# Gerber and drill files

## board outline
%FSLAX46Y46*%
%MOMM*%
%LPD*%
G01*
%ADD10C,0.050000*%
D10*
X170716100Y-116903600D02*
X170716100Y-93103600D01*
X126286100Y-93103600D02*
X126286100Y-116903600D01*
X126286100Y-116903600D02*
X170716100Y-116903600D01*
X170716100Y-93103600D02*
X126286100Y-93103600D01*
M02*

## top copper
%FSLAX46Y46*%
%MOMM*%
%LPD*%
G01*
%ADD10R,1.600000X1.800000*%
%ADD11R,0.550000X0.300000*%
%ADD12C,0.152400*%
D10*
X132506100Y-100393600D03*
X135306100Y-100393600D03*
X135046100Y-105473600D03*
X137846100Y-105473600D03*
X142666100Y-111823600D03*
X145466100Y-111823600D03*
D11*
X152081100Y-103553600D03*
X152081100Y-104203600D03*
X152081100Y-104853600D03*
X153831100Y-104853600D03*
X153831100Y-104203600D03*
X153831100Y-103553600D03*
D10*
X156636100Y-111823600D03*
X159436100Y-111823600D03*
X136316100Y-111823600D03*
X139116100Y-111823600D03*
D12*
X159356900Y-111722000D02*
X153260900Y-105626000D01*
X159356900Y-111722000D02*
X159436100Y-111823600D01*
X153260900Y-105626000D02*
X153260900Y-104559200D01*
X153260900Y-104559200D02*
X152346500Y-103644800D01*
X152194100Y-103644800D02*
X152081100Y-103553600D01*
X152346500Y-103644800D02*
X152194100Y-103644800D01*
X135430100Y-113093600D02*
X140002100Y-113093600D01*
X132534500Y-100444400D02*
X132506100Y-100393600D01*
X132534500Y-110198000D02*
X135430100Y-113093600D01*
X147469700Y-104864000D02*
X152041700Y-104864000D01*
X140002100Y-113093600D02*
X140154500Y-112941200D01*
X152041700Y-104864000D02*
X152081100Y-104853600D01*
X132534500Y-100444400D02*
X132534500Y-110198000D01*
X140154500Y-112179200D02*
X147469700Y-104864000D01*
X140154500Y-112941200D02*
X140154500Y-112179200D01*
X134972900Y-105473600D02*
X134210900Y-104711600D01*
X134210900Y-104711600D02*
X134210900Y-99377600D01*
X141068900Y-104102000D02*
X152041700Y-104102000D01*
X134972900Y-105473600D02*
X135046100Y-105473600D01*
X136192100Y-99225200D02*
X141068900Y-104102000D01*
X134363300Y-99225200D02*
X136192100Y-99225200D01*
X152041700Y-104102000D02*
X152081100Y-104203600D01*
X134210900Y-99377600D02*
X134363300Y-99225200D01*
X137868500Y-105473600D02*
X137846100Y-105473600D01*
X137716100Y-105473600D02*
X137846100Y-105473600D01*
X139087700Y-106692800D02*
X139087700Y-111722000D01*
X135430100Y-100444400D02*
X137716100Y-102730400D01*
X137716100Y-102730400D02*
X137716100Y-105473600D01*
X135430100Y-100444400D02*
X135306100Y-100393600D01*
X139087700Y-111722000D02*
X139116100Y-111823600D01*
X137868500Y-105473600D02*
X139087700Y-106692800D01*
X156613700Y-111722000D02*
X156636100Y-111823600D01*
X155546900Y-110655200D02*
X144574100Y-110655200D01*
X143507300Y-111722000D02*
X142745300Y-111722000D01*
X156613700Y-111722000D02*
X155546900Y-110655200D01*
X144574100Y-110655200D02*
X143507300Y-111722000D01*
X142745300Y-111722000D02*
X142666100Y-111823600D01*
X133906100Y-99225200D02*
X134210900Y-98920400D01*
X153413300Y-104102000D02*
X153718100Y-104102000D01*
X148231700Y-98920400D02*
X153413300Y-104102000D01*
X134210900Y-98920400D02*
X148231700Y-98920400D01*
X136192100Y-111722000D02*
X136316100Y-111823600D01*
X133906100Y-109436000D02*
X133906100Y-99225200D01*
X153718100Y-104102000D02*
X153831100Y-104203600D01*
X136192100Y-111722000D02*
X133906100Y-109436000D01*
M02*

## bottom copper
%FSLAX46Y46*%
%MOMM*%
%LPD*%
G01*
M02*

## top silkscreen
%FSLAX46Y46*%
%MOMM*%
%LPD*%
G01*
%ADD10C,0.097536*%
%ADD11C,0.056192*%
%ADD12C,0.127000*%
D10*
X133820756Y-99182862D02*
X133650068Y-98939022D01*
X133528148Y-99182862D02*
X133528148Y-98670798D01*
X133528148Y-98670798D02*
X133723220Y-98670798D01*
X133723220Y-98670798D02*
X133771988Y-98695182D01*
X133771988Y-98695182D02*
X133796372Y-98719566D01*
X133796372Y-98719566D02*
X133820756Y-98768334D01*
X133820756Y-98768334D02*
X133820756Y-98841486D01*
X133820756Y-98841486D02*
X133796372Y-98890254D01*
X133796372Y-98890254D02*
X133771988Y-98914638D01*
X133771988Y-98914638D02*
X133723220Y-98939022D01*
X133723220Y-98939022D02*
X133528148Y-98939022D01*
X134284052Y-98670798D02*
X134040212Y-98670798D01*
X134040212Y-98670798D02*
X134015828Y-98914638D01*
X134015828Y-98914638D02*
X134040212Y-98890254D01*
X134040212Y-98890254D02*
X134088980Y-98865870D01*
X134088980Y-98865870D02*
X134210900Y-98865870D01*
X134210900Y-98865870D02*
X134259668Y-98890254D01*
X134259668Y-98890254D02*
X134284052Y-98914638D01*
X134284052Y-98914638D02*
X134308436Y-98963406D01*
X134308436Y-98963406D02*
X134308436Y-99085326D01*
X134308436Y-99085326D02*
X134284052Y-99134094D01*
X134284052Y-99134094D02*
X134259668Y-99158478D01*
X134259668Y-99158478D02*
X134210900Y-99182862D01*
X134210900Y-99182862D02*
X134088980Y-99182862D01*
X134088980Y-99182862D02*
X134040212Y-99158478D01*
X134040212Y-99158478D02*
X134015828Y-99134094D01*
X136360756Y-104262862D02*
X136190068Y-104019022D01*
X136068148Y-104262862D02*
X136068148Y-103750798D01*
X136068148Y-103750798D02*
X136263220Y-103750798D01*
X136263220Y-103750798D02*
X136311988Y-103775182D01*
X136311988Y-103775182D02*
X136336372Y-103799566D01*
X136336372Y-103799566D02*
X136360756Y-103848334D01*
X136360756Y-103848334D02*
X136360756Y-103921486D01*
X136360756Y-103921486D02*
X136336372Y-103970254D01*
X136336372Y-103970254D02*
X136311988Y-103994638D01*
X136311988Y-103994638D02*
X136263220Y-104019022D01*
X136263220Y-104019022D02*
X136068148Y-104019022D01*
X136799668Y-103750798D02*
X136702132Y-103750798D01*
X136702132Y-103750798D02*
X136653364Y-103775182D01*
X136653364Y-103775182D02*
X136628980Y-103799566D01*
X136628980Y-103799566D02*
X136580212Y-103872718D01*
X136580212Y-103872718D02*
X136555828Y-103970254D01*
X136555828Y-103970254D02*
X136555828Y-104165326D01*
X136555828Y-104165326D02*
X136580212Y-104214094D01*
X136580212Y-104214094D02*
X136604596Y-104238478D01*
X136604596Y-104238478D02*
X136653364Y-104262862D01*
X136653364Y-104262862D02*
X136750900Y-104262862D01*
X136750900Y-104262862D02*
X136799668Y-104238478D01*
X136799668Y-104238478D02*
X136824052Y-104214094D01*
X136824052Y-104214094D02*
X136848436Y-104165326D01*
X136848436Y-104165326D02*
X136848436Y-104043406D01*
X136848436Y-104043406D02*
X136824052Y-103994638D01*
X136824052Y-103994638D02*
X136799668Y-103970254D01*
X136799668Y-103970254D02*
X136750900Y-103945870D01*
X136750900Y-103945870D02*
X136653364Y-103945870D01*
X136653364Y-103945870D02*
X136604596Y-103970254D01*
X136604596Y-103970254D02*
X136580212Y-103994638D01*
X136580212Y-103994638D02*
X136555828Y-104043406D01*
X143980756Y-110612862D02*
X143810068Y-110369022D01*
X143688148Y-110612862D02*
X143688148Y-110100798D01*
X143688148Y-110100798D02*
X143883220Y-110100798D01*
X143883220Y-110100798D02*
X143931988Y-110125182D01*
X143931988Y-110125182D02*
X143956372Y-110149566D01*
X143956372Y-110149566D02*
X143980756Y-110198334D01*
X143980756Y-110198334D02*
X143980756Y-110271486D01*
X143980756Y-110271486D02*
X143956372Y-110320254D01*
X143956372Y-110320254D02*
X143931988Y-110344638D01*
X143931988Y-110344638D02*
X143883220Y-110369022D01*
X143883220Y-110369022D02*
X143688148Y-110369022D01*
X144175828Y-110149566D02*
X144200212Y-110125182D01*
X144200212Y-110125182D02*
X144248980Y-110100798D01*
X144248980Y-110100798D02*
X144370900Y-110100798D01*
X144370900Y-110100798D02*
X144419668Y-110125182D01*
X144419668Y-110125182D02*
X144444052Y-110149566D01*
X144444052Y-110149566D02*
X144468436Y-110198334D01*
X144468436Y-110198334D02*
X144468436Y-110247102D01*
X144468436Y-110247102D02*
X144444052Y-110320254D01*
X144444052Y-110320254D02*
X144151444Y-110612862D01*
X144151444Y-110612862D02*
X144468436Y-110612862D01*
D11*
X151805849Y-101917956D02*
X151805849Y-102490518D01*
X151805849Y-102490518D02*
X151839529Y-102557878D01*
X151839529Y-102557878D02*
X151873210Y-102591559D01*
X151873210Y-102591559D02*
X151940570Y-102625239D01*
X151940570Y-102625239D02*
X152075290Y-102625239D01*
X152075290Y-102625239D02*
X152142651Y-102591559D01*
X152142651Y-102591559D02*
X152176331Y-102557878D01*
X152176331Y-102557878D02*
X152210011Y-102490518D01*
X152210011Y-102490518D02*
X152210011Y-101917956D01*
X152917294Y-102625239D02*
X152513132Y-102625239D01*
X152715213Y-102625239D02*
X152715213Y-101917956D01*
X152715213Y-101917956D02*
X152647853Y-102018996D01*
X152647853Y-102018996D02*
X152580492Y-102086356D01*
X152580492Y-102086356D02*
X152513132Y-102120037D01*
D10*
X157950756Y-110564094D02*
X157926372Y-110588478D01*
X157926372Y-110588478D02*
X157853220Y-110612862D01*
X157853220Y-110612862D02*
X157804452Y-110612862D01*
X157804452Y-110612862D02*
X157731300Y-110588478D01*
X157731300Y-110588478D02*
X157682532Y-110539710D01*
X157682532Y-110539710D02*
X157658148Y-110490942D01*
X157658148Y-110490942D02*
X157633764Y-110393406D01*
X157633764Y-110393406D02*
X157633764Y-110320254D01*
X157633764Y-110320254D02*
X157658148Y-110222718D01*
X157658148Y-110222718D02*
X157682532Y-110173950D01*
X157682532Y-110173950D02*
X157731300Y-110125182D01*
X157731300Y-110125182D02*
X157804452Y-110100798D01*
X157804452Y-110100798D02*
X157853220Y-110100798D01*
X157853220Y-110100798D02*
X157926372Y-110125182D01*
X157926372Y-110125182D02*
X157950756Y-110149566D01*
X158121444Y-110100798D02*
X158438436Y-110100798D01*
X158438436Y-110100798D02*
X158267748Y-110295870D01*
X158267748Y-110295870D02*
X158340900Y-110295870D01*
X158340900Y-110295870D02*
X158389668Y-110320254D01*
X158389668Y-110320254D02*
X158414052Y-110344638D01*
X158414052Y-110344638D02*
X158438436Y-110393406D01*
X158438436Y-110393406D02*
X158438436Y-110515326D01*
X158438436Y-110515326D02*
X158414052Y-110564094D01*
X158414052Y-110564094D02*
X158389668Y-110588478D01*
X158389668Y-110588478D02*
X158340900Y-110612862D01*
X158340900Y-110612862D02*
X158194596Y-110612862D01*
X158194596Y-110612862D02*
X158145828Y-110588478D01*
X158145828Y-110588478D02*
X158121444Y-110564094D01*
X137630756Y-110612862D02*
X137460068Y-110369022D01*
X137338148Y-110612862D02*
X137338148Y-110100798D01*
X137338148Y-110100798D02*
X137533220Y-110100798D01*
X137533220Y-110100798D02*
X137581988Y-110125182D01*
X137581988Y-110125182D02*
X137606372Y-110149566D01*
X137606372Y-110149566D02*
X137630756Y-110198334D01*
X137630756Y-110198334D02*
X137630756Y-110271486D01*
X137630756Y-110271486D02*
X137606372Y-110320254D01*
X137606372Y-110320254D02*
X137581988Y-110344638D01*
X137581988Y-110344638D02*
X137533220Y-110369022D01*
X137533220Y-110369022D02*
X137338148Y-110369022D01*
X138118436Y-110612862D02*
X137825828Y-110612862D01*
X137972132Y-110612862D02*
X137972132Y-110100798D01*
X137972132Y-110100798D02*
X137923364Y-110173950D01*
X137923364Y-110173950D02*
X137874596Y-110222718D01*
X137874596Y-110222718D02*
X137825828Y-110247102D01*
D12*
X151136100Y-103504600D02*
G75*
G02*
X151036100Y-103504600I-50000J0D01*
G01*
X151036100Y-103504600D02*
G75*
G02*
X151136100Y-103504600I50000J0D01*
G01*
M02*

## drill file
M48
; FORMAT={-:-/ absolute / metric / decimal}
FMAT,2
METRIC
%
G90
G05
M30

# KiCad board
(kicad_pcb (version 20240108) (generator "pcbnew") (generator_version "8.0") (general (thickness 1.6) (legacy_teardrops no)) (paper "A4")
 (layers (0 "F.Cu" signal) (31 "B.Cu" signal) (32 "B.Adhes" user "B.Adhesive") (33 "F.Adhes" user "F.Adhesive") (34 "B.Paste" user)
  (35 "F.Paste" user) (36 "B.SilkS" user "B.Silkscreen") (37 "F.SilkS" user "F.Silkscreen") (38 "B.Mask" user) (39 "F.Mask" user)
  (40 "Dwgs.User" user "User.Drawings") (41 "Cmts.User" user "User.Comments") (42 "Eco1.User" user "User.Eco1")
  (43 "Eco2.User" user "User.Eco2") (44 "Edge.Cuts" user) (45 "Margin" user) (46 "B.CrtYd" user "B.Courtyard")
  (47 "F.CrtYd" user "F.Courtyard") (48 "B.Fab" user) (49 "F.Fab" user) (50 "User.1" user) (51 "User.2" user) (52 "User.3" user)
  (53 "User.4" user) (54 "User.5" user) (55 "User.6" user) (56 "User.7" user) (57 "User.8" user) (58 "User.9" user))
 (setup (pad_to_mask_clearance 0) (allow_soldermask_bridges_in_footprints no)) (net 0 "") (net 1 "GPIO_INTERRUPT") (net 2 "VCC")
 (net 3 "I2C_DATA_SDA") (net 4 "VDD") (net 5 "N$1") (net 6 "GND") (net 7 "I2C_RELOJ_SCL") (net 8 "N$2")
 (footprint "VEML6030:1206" (layer "F.Cu") (at 133.9061 100.3936)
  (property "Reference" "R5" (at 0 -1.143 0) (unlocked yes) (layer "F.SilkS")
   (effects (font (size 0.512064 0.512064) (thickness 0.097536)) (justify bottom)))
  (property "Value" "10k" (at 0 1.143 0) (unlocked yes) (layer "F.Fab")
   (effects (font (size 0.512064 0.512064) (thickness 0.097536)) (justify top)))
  (pad "1" smd rect (at -1.4 0) (size 1.6 1.8) (layers "F.Cu" "F.Paste" "F.Mask") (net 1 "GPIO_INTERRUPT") (solder_mask_margin 0.1016)
   (thermal_bridge_angle 0))
  (pad "2" smd rect (at 1.4 0) (size 1.6 1.8) (layers "F.Cu" "F.Paste" "F.Mask") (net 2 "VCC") (solder_mask_margin 0.1016)
   (thermal_bridge_angle 0)))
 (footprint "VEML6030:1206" (layer "F.Cu") (at 136.4461 105.4736)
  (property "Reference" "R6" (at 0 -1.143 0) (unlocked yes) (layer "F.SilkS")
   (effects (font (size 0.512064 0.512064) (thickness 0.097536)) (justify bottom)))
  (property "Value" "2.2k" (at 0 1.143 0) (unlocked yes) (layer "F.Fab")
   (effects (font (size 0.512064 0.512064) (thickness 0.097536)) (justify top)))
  (pad "1" smd rect (at -1.4 0) (size 1.6 1.8) (layers "F.Cu" "F.Paste" "F.Mask") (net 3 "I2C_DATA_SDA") (solder_mask_margin 0.1016)
   (thermal_bridge_angle 0))
  (pad "2" smd rect (at 1.4 0) (size 1.6 1.8) (layers "F.Cu" "F.Paste" "F.Mask") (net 2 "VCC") (solder_mask_margin 0.1016)
   (thermal_bridge_angle 0)))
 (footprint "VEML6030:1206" (layer "F.Cu") (at 144.0661 111.8236)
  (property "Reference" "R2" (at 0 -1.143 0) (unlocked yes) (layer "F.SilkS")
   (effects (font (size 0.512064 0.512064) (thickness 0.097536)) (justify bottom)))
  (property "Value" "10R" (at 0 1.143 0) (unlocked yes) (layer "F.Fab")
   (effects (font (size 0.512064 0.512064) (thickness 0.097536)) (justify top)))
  (pad "1" smd rect (at -1.4 0) (size 1.6 1.8) (layers "F.Cu" "F.Paste" "F.Mask") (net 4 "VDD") (solder_mask_margin 0.1016)
   (thermal_bridge_angle 0))
  (pad "2" smd rect (at 1.4 0) (size 1.6 1.8) (layers "F.Cu" "F.Paste" "F.Mask") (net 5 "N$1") (solder_mask_margin 0.1016)
   (thermal_bridge_angle 0)))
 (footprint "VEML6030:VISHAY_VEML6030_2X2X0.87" (layer "F.Cu") (at 152.9561 104.2036)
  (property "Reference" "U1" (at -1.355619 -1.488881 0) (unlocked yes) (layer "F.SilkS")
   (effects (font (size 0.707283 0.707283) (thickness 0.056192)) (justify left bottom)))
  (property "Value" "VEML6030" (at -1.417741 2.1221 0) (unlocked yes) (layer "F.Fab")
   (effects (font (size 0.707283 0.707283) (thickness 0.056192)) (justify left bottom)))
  (fp_circle (center -1.87 -0.699) (end -1.82 -0.699) (stroke (width 0.127) (type solid)) (fill none) (layer "F.SilkS"))
  (pad "1" smd rect (at -0.875 -0.65) (size 0.55 0.3) (layers "F.Cu" "F.Paste" "F.Mask") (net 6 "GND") (solder_mask_margin 0.1016)
   (thermal_bridge_angle 0))
  (pad "2" smd rect (at -0.875 0) (size 0.55 0.3) (layers "F.Cu" "F.Paste" "F.Mask") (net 3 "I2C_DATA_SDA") (solder_mask_margin 0.1016)
   (thermal_bridge_angle 0))
  (pad "3" smd rect (at -0.875 0.65) (size 0.55 0.3) (layers "F.Cu" "F.Paste" "F.Mask") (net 1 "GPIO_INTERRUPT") (solder_mask_margin 0.1016)
   (thermal_bridge_angle 0))
  (pad "4" smd rect (at 0.875 0.65) (size 0.55 0.3) (layers "F.Cu" "F.Paste" "F.Mask") (solder_mask_margin 0.1016) (thermal_bridge_angle 0))
  (pad "5" smd rect (at 0.875 0) (size 0.55 0.3) (layers "F.Cu" "F.Paste" "F.Mask") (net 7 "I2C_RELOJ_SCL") (solder_mask_margin 0.1016)
   (thermal_bridge_angle 0))
  (pad "6" smd rect (at 0.875 -0.65) (size 0.55 0.3) (layers "F.Cu" "F.Paste" "F.Mask") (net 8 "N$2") (solder_mask_margin 0.1016)
   (thermal_bridge_angle 0)))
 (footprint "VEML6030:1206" (layer "F.Cu") (at 158.0361 111.8236)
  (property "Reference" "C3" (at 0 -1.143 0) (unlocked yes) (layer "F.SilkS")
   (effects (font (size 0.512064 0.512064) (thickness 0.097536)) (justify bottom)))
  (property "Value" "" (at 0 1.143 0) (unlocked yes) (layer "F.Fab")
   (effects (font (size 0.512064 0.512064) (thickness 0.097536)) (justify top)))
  (pad "1" smd rect (at -1.4 0) (size 1.6 1.8) (layers "F.Cu" "F.Paste" "F.Mask") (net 4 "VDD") (solder_mask_margin 0.1016)
   (thermal_bridge_angle 0))
  (pad "2" smd rect (at 1.4 0) (size 1.6 1.8) (layers "F.Cu" "F.Paste" "F.Mask") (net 6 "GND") (solder_mask_margin 0.1016)
   (thermal_bridge_angle 0)))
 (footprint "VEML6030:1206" (layer "F.Cu") (at 137.7161 111.8236)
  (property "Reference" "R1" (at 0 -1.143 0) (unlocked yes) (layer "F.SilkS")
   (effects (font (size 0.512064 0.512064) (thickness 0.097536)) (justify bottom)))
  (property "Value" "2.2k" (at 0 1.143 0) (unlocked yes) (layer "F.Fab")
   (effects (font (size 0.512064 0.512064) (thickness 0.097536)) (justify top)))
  (pad "1" smd rect (at -1.4 0) (size 1.6 1.8) (layers "F.Cu" "F.Paste" "F.Mask") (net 7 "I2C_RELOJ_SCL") (solder_mask_margin 0.1016)
   (thermal_bridge_angle 0))
  (pad "2" smd rect (at 1.4 0) (size 1.6 1.8) (layers "F.Cu" "F.Paste" "F.Mask") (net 2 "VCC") (solder_mask_margin 0.1016)
   (thermal_bridge_angle 0)))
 (gr_line (start 170.7161 116.9036) (end 170.7161 93.1036) (stroke (width 0.05) (type solid)) (layer "Edge.Cuts"))
 (gr_line (start 126.2861 93.1036) (end 126.2861 116.9036) (stroke (width 0.05) (type solid)) (layer "Edge.Cuts"))
 (gr_line (start 126.2861 116.9036) (end 170.7161 116.9036) (stroke (width 0.05) (type solid)) (layer "Edge.Cuts"))
 (gr_line (start 170.7161 93.1036) (end 126.2861 93.1036) (stroke (width 0.05) (type solid)) (layer "Edge.Cuts"))
 (segment (start 159.3569 111.722) (end 153.2609 105.626) (width 0.1524) (layer "F.Cu") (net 6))
 (segment (start 159.3569 111.722) (end 159.4361 111.8236) (width 0.1524) (layer "F.Cu") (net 6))
 (segment (start 153.2609 105.626) (end 153.2609 104.5592) (width 0.1524) (layer "F.Cu") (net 6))
 (segment (start 153.2609 104.5592) (end 152.3465 103.6448) (width 0.1524) (layer "F.Cu") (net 6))
 (segment (start 152.1941 103.6448) (end 152.0811 103.5536) (width 0.1524) (layer "F.Cu") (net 6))
 (segment (start 152.3465 103.6448) (end 152.1941 103.6448) (width 0.1524) (layer "F.Cu") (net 6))
 (segment (start 135.4301 113.0936) (end 140.0021 113.0936) (width 0.1524) (layer "F.Cu") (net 1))
 (segment (start 132.5345 100.4444) (end 132.5061 100.3936) (width 0.1524) (layer "F.Cu") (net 1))
 (segment (start 132.5345 110.198) (end 135.4301 113.0936) (width 0.1524) (layer "F.Cu") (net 1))
 (segment (start 147.4697 104.864) (end 152.0417 104.864) (width 0.1524) (layer "F.Cu") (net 1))
 (segment (start 140.0021 113.0936) (end 140.1545 112.9412) (width 0.1524) (layer "F.Cu") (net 1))
 (segment (start 152.0417 104.864) (end 152.0811 104.8536) (width 0.1524) (layer "F.Cu") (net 1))
 (segment (start 132.5345 100.4444) (end 132.5345 110.198) (width 0.1524) (layer "F.Cu") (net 1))
 (segment (start 140.1545 112.1792) (end 147.4697 104.864) (width 0.1524) (layer "F.Cu") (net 1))
 (segment (start 140.1545 112.9412) (end 140.1545 112.1792) (width 0.1524) (layer "F.Cu") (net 1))
 (segment (start 134.9729 105.4736) (end 134.2109 104.7116) (width 0.1524) (layer "F.Cu") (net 3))
 (segment (start 134.2109 104.7116) (end 134.2109 99.3776) (width 0.1524) (layer "F.Cu") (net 3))
 (segment (start 141.0689 104.102) (end 152.0417 104.102) (width 0.1524) (layer "F.Cu") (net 3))
 (segment (start 134.9729 105.4736) (end 135.0461 105.4736) (width 0.1524) (layer "F.Cu") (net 3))
 (segment (start 136.1921 99.2252) (end 141.0689 104.102) (width 0.1524) (layer "F.Cu") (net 3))
 (segment (start 134.3633 99.2252) (end 136.1921 99.2252) (width 0.1524) (layer "F.Cu") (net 3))
 (segment (start 152.0417 104.102) (end 152.0811 104.2036) (width 0.1524) (layer "F.Cu") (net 3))
 (segment (start 134.2109 99.3776) (end 134.3633 99.2252) (width 0.1524) (layer "F.Cu") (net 3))
 (segment (start 137.8685 105.4736) (end 137.8461 105.4736) (width 0.1524) (layer "F.Cu") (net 2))
 (segment (start 137.7161 105.4736) (end 137.8461 105.4736) (width 0.1524) (layer "F.Cu") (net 2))
 (segment (start 139.0877 106.6928) (end 139.0877 111.722) (width 0.1524) (layer "F.Cu") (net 2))
 (segment (start 135.4301 100.4444) (end 137.7161 102.7304) (width 0.1524) (layer "F.Cu") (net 2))
 (segment (start 137.7161 102.7304) (end 137.7161 105.4736) (width 0.1524) (layer "F.Cu") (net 2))
 (segment (start 135.4301 100.4444) (end 135.3061 100.3936) (width 0.1524) (layer "F.Cu") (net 2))
 (segment (start 139.0877 111.722) (end 139.1161 111.8236) (width 0.1524) (layer "F.Cu") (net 2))
 (segment (start 137.8685 105.4736) (end 139.0877 106.6928) (width 0.1524) (layer "F.Cu") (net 2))
 (segment (start 156.6137 111.722) (end 156.6361 111.8236) (width 0.1524) (layer "F.Cu") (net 4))
 (segment (start 155.5469 110.6552) (end 144.5741 110.6552) (width 0.1524) (layer "F.Cu") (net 4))
 (segment (start 143.5073 111.722) (end 142.7453 111.722) (width 0.1524) (layer "F.Cu") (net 4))
 (segment (start 156.6137 111.722) (end 155.5469 110.6552) (width 0.1524) (layer "F.Cu") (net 4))
 (segment (start 144.5741 110.6552) (end 143.5073 111.722) (width 0.1524) (layer "F.Cu") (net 4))
 (segment (start 142.7453 111.722) (end 142.6661 111.8236) (width 0.1524) (layer "F.Cu") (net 4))
 (segment (start 133.9061 99.2252) (end 134.2109 98.9204) (width 0.1524) (layer "F.Cu") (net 7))
 (segment (start 153.4133 104.102) (end 153.7181 104.102) (width 0.1524) (layer "F.Cu") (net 7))
 (segment (start 148.2317 98.9204) (end 153.4133 104.102) (width 0.1524) (layer "F.Cu") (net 7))
 (segment (start 134.2109 98.9204) (end 148.2317 98.9204) (width 0.1524) (layer "F.Cu") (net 7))
 (segment (start 136.1921 111.722) (end 136.3161 111.8236) (width 0.1524) (layer "F.Cu") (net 7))
 (segment (start 133.9061 109.436) (end 133.9061 99.2252) (width 0.1524) (layer "F.Cu") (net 7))
 (segment (start 153.7181 104.102) (end 153.8311 104.2036) (width 0.1524) (layer "F.Cu") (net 7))
 (segment (start 136.1921 111.722) (end 133.9061 109.436) (width 0.1524) (layer "F.Cu") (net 7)))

